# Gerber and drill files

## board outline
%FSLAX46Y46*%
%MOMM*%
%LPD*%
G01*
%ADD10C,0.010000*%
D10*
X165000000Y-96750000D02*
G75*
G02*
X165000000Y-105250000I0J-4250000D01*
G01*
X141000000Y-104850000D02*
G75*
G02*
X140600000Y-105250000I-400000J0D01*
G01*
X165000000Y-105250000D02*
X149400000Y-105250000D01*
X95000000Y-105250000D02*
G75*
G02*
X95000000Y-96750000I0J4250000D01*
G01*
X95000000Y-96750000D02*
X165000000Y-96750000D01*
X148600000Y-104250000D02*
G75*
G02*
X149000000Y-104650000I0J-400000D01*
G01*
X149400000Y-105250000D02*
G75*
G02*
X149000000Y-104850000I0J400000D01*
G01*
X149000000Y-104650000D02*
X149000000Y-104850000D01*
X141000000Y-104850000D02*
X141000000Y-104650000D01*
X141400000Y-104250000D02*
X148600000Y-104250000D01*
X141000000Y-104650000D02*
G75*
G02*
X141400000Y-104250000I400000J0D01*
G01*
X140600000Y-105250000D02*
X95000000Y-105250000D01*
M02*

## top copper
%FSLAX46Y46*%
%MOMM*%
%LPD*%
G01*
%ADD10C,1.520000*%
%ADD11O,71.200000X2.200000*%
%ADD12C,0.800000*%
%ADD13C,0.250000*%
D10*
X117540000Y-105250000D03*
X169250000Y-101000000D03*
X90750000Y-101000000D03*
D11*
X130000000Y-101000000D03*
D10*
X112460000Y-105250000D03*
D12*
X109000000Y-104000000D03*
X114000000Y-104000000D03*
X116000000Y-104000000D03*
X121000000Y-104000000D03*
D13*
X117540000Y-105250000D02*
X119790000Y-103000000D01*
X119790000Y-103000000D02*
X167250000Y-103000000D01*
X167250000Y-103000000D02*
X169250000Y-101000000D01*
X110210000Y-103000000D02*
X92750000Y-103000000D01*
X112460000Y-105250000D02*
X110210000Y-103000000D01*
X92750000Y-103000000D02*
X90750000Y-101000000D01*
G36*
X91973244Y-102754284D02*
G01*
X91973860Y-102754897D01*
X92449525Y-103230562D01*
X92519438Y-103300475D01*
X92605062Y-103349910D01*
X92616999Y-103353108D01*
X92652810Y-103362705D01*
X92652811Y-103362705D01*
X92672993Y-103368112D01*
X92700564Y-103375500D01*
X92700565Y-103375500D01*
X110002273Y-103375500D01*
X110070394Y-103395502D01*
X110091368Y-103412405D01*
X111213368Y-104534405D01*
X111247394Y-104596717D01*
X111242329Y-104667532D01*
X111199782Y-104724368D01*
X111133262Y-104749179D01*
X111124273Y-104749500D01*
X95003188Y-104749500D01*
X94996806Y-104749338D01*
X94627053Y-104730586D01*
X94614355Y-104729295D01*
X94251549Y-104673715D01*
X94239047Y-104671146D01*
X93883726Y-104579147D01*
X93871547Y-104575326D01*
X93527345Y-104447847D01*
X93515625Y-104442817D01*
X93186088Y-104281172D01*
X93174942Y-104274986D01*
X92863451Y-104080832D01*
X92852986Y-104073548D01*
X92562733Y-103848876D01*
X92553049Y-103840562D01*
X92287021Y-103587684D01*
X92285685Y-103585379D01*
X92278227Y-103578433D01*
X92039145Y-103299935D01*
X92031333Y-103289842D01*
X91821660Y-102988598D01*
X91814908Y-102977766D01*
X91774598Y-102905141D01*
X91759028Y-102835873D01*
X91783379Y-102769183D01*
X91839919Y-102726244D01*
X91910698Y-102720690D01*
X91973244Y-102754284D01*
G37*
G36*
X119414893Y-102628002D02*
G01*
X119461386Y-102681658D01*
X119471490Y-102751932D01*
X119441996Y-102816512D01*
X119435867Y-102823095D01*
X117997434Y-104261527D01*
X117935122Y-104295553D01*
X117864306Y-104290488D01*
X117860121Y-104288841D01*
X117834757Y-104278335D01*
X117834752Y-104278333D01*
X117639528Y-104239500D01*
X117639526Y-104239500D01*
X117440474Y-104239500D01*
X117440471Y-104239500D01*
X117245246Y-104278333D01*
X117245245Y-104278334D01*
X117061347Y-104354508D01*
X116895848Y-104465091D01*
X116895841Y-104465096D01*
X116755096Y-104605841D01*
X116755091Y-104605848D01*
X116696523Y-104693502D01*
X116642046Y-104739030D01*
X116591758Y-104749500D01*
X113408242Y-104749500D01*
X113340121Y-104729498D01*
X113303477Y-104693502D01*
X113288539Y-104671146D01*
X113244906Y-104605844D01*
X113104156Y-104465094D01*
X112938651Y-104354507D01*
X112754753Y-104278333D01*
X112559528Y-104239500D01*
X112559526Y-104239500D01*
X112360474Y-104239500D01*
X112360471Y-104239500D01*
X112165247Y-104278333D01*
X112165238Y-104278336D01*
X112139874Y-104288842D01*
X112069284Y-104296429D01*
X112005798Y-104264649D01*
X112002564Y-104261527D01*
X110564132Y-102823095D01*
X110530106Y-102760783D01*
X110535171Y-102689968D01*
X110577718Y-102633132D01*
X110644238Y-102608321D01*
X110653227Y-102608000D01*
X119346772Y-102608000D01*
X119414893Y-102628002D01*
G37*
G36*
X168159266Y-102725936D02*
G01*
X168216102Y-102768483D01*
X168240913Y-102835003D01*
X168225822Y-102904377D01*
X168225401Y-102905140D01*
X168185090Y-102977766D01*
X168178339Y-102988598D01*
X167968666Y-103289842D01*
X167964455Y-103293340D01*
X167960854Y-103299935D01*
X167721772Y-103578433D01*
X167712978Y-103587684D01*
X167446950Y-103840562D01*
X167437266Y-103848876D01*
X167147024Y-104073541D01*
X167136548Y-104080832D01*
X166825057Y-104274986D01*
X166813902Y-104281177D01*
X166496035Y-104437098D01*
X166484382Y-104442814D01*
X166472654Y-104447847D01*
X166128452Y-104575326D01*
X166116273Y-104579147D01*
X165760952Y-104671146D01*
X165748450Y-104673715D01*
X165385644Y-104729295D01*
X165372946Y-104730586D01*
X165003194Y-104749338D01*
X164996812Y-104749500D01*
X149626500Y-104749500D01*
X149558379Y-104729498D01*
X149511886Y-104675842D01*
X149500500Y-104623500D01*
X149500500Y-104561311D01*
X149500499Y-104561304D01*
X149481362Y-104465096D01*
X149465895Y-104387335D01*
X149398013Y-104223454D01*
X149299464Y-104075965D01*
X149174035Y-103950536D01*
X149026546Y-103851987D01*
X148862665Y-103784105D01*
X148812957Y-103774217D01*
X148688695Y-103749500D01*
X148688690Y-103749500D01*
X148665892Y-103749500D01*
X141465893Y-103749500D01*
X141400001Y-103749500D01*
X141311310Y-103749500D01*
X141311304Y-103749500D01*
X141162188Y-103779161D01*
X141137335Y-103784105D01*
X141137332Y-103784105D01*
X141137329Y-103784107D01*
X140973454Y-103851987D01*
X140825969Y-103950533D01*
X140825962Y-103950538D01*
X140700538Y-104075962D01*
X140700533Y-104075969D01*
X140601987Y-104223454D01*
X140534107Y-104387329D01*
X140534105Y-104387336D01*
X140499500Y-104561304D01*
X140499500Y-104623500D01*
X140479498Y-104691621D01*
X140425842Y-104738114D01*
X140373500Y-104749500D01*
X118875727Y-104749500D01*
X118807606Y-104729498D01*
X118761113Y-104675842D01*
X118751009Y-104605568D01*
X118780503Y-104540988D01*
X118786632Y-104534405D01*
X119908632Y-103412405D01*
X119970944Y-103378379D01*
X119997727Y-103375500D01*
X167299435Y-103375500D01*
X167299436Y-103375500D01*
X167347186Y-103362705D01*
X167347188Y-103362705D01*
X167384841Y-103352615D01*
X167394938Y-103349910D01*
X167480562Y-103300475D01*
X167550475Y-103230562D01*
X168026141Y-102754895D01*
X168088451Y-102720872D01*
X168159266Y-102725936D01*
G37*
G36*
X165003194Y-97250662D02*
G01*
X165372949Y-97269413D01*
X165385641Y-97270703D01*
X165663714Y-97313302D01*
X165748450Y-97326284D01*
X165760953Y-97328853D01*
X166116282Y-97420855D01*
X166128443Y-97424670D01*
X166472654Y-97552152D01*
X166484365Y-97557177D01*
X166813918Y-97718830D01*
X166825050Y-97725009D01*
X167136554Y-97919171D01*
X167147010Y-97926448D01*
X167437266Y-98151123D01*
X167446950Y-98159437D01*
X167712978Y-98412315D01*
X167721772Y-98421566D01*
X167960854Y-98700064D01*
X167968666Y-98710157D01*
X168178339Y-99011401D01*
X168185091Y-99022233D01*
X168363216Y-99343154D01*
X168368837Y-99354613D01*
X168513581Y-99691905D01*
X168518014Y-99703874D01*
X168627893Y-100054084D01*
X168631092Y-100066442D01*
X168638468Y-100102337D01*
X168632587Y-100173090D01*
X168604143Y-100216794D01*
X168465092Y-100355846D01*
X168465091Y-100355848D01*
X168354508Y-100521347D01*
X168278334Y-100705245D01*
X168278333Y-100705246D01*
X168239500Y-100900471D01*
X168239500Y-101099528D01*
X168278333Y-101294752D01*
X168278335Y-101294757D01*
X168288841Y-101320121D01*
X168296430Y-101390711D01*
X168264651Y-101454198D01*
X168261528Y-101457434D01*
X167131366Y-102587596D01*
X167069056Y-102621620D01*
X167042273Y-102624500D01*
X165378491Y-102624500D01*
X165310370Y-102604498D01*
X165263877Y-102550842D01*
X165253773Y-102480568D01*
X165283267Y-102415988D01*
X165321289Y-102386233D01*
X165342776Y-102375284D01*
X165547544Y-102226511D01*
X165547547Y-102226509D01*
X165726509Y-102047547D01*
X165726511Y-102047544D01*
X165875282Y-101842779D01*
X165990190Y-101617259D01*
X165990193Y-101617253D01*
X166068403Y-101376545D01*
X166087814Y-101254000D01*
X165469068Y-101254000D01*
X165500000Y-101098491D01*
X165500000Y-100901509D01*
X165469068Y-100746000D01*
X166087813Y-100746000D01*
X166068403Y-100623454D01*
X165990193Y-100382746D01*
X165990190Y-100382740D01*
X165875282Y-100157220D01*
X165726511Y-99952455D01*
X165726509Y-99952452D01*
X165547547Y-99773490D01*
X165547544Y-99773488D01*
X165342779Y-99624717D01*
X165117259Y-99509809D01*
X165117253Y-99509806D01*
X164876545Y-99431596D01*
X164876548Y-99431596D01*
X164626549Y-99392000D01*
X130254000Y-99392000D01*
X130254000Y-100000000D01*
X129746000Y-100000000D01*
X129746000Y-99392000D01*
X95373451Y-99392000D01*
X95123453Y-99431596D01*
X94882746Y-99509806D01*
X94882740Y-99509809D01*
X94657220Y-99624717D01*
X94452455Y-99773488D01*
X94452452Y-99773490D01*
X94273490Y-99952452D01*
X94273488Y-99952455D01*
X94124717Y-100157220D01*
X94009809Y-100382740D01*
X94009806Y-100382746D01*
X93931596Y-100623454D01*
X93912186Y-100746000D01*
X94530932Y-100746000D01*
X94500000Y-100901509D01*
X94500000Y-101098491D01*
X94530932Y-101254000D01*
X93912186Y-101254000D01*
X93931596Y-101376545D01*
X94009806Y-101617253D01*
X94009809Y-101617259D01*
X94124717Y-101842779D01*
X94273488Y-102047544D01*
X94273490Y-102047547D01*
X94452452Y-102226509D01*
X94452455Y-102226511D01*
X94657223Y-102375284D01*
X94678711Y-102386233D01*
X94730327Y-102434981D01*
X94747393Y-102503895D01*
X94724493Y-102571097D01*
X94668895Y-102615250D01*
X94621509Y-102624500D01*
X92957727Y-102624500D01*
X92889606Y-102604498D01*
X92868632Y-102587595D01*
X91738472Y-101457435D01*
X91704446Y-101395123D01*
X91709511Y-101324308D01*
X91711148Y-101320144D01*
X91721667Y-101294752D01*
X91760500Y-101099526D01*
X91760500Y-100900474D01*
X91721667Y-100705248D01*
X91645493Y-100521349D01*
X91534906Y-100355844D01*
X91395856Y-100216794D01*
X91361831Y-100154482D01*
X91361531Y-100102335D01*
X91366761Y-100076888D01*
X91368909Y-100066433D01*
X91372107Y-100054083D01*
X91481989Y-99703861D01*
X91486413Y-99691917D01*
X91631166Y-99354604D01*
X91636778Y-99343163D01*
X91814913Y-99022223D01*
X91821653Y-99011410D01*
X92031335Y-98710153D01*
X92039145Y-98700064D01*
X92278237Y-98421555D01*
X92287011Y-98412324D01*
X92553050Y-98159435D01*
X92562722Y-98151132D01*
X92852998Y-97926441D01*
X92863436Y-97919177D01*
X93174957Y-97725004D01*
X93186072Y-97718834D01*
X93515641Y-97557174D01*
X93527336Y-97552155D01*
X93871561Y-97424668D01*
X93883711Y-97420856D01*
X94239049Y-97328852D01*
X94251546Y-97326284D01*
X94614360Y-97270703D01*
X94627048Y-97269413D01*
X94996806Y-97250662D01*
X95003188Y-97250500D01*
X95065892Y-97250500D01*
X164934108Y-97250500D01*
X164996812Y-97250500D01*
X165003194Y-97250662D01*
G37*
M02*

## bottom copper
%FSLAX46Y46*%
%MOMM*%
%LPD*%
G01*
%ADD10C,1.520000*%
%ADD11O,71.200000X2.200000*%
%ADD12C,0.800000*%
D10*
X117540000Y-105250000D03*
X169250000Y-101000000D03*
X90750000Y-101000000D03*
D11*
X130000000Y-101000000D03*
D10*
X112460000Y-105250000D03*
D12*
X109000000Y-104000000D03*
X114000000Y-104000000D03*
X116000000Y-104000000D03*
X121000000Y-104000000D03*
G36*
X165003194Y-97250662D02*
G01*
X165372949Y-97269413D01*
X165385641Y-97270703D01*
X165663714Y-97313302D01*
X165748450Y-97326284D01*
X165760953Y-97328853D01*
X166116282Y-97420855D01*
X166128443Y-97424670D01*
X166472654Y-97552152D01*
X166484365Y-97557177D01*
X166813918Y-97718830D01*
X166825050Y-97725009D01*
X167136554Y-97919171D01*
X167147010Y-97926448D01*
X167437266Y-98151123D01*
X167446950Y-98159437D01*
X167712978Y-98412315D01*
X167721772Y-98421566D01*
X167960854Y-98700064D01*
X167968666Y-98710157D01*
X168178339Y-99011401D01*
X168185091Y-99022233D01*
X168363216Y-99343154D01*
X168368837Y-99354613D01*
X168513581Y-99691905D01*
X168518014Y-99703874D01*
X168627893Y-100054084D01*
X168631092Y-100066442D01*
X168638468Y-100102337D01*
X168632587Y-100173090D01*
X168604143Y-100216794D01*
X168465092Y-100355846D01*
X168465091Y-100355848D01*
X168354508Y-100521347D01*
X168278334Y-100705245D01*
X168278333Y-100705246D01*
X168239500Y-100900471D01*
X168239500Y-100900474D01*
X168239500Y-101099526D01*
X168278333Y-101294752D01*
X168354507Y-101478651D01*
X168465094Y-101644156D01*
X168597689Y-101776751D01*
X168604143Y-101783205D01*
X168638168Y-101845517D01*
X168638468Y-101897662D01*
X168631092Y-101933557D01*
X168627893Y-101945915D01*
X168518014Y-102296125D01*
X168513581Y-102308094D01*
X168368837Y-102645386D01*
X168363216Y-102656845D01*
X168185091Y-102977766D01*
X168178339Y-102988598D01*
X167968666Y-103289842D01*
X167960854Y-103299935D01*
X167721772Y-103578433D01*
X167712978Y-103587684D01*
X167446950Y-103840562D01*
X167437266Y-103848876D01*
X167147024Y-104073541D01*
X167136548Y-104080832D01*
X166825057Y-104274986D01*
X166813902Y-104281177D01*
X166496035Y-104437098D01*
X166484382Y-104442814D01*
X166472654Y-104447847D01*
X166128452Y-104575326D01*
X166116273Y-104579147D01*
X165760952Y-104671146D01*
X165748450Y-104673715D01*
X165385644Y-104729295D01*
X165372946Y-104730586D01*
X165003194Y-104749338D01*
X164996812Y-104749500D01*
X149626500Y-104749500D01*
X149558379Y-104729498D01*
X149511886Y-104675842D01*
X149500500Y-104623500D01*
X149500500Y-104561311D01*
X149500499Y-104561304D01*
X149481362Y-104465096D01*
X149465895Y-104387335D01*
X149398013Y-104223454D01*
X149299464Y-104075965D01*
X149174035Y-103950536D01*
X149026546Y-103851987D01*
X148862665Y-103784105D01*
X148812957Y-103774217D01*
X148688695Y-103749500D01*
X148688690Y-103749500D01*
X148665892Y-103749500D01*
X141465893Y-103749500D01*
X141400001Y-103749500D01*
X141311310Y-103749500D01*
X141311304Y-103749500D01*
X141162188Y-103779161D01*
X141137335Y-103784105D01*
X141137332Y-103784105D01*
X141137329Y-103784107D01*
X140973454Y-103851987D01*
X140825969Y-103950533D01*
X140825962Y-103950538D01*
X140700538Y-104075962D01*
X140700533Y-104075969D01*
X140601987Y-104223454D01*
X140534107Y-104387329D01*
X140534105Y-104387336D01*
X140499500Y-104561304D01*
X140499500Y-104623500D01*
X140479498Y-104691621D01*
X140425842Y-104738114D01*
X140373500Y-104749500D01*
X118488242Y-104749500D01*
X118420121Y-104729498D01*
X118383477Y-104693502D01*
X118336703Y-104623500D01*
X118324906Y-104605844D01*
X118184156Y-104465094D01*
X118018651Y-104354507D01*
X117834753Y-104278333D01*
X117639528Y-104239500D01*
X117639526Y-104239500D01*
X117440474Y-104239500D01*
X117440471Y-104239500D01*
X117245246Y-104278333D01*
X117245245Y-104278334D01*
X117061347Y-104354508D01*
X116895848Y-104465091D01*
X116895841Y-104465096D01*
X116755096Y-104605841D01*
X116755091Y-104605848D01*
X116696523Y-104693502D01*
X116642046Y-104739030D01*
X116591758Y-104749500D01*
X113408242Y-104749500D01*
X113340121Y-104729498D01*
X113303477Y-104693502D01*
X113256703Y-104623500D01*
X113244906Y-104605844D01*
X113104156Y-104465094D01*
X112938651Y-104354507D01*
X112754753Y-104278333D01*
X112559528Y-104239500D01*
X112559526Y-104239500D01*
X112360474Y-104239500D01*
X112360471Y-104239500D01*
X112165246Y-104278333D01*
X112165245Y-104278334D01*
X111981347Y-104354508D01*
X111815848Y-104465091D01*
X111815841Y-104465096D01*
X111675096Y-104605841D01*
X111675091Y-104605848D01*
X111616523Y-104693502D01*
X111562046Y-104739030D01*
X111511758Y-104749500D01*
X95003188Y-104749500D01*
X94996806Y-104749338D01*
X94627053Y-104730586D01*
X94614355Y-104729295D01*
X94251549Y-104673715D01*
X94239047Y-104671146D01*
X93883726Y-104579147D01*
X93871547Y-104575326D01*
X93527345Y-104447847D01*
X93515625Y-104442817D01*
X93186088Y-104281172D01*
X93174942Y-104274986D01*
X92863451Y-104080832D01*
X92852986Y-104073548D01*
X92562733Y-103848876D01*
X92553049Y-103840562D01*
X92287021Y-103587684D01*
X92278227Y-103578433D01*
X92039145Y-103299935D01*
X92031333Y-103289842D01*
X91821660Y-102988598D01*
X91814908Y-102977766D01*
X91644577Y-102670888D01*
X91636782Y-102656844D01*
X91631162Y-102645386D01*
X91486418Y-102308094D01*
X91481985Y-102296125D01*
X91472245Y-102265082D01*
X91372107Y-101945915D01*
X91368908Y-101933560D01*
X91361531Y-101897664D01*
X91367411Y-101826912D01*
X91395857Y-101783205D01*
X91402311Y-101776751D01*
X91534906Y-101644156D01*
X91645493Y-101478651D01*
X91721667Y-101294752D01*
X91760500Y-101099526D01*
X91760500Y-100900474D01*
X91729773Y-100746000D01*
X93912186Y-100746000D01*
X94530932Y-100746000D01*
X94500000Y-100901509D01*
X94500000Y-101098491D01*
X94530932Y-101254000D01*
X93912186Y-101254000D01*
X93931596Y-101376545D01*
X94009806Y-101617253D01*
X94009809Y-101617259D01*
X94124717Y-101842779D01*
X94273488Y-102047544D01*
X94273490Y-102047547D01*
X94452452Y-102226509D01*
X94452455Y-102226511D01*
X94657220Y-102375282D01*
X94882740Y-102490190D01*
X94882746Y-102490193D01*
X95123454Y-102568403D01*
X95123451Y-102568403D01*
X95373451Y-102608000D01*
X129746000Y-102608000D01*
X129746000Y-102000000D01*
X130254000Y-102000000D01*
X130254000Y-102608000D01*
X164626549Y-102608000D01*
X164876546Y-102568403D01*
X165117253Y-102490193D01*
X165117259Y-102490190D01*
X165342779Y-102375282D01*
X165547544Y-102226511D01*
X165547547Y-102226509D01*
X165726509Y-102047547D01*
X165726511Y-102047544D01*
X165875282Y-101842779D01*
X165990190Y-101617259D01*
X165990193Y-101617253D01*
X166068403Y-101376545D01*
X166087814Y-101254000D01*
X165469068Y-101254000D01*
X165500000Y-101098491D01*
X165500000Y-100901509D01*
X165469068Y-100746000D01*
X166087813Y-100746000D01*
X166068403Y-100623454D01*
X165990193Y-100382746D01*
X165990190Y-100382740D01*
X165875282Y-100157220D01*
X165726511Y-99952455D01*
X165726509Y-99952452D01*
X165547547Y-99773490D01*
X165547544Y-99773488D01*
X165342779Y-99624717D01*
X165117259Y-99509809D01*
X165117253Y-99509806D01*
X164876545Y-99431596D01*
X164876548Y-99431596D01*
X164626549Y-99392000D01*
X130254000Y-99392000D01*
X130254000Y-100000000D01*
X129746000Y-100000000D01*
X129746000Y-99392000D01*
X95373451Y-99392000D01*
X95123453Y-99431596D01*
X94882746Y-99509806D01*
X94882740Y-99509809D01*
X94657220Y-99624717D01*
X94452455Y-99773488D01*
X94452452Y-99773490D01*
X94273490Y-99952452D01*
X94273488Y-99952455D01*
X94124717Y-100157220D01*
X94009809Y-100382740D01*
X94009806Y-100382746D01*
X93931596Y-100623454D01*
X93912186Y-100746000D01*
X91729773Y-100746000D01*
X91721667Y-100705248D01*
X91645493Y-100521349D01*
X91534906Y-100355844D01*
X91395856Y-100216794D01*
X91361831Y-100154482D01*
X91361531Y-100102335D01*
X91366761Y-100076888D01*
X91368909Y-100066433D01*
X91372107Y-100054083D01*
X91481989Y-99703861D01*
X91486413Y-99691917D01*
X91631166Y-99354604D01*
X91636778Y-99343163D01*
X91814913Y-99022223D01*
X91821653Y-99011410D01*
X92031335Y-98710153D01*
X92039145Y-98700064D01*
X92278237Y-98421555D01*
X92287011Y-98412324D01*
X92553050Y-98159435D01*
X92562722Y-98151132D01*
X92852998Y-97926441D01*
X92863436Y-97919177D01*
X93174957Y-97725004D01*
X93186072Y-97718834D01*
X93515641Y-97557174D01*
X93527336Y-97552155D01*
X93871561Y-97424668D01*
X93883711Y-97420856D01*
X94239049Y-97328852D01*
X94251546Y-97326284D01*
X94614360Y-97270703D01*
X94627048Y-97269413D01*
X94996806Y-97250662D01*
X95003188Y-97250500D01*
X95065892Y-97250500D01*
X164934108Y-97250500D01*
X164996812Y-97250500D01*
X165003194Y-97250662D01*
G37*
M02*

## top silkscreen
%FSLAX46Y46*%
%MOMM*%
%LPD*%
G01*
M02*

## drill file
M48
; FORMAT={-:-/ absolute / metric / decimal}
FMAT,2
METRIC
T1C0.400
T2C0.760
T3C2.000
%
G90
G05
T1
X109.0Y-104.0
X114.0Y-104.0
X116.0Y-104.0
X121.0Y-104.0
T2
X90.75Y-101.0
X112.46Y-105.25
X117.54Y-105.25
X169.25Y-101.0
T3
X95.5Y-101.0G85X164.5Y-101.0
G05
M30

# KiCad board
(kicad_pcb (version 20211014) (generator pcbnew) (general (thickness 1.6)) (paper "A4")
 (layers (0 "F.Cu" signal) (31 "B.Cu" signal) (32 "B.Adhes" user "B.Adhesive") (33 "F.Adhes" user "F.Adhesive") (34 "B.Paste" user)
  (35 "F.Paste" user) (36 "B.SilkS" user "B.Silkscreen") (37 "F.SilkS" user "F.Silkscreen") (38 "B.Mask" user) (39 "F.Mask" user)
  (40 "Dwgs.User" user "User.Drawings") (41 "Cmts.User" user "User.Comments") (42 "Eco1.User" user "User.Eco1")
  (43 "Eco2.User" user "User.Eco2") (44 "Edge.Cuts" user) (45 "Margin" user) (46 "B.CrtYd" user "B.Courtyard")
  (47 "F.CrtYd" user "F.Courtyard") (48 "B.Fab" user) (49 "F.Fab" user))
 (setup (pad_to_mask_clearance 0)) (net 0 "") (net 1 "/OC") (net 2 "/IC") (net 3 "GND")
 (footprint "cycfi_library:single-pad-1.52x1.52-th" (layer "F.Cu") (at 117.54 105.25 180)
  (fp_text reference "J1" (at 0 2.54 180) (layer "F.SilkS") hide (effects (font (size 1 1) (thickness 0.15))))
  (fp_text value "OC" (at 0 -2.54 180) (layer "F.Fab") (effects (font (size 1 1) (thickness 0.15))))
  (pad "1" thru_hole circle (at 0 0 180) (size 1.52 1.52) (drill 0.76) (layers *.Cu *.Mask) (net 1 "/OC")))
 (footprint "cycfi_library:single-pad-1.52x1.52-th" (layer "F.Cu") (at 169.25 101 180)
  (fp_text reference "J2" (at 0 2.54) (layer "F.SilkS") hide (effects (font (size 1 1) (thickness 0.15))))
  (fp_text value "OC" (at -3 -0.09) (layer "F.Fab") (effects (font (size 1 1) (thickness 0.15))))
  (pad "1" thru_hole circle (at 0 0 180) (size 1.52 1.52) (drill 0.76) (layers *.Cu *.Mask) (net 1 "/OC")))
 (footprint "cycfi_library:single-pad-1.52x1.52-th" (layer "F.Cu") (at 90.75 101)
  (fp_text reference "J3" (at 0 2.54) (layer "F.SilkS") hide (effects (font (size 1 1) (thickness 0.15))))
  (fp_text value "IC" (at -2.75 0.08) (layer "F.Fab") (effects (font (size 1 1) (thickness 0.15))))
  (pad "1" thru_hole circle (at 0 0) (size 1.52 1.52) (drill 0.76) (layers *.Cu *.Mask) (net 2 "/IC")))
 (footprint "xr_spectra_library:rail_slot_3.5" (layer "F.Cu") (at 129.75 101)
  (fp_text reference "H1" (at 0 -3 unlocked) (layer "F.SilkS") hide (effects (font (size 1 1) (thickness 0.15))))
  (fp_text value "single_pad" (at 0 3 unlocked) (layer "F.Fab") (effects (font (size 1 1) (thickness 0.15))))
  (pad "1" thru_hole oval (at 0.25 0) (size 71.2 2.2) (drill oval 71 2) (layers *.Cu *.Mask) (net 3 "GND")))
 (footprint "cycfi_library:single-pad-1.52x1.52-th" (layer "F.Cu") (at 112.46 105.25)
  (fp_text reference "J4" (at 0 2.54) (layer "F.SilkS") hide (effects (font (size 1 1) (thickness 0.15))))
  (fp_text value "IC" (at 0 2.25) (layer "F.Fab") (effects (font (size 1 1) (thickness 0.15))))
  (pad "1" thru_hole circle (at 0 0) (size 1.52 1.52) (drill 0.76) (layers *.Cu *.Mask) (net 2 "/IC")))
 (gr_arc (start 165 96.75) (mid 169.25 101) (end 165 105.25) (layer "Edge.Cuts") (width 0.01))
 (gr_arc (start 141 104.85) (mid 140.882843 105.132843) (end 140.6 105.25) (layer "Edge.Cuts") (width 0.01))
 (gr_line (start 165 105.25) (end 149.4 105.25) (layer "Edge.Cuts") (width 0.01))
 (gr_arc (start 95 105.25) (mid 90.75 101) (end 95 96.75) (layer "Edge.Cuts") (width 0.01))
 (gr_line (start 95 96.75) (end 165 96.75) (layer "Edge.Cuts") (width 0.01))
 (gr_arc (start 148.6 104.25) (mid 148.882843 104.367157) (end 149 104.65) (layer "Edge.Cuts") (width 0.01))
 (gr_arc (start 149.4 105.25) (mid 149.117157 105.132843) (end 149 104.85) (layer "Edge.Cuts") (width 0.01))
 (gr_line (start 149 104.65) (end 149 104.85) (layer "Edge.Cuts") (width 0.01))
 (gr_line (start 141 104.85) (end 141 104.65) (layer "Edge.Cuts") (width 0.01))
 (gr_line (start 141.4 104.25) (end 148.6 104.25) (layer "Edge.Cuts") (width 0.01))
 (gr_arc (start 141 104.65) (mid 141.117157 104.367157) (end 141.4 104.25) (layer "Edge.Cuts") (width 0.01))
 (gr_line (start 140.6 105.25) (end 95 105.25) (layer "Edge.Cuts") (width 0.01))
 (via (at 109 104) (size 0.8) (drill 0.4) (layers "F.Cu" "B.Cu") (free) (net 3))
 (via (at 114 104) (size 0.8) (drill 0.4) (layers "F.Cu" "B.Cu") (free) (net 3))
 (via (at 116 104) (size 0.8) (drill 0.4) (layers "F.Cu" "B.Cu") (free) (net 3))
 (via (at 121 104) (size 0.8) (drill 0.4) (layers "F.Cu" "B.Cu") (free) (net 3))
 (segment (start 117.54 105.25) (end 119.79 103) (width 0.25) (layer "F.Cu") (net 1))
 (segment (start 119.79 103) (end 167.25 103) (width 0.25) (layer "F.Cu") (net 1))
 (segment (start 167.25 103) (end 169.25 101) (width 0.25) (layer "F.Cu") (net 1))
 (segment (start 110.21 103) (end 92.75 103) (width 0.25) (layer "F.Cu") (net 2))
 (segment (start 112.46 105.25) (end 110.21 103) (width 0.25) (layer "F.Cu") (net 2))
 (segment (start 92.75 103) (end 90.75 101) (width 0.25) (layer "F.Cu") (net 2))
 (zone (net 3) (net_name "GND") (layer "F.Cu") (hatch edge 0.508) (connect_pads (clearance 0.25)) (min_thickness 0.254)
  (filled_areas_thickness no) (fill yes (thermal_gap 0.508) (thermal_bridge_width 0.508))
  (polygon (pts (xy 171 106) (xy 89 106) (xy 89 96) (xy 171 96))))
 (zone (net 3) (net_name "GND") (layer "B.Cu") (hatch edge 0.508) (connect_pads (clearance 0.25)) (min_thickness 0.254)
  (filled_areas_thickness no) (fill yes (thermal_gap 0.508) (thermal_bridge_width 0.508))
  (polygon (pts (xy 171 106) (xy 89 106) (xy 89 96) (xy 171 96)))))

